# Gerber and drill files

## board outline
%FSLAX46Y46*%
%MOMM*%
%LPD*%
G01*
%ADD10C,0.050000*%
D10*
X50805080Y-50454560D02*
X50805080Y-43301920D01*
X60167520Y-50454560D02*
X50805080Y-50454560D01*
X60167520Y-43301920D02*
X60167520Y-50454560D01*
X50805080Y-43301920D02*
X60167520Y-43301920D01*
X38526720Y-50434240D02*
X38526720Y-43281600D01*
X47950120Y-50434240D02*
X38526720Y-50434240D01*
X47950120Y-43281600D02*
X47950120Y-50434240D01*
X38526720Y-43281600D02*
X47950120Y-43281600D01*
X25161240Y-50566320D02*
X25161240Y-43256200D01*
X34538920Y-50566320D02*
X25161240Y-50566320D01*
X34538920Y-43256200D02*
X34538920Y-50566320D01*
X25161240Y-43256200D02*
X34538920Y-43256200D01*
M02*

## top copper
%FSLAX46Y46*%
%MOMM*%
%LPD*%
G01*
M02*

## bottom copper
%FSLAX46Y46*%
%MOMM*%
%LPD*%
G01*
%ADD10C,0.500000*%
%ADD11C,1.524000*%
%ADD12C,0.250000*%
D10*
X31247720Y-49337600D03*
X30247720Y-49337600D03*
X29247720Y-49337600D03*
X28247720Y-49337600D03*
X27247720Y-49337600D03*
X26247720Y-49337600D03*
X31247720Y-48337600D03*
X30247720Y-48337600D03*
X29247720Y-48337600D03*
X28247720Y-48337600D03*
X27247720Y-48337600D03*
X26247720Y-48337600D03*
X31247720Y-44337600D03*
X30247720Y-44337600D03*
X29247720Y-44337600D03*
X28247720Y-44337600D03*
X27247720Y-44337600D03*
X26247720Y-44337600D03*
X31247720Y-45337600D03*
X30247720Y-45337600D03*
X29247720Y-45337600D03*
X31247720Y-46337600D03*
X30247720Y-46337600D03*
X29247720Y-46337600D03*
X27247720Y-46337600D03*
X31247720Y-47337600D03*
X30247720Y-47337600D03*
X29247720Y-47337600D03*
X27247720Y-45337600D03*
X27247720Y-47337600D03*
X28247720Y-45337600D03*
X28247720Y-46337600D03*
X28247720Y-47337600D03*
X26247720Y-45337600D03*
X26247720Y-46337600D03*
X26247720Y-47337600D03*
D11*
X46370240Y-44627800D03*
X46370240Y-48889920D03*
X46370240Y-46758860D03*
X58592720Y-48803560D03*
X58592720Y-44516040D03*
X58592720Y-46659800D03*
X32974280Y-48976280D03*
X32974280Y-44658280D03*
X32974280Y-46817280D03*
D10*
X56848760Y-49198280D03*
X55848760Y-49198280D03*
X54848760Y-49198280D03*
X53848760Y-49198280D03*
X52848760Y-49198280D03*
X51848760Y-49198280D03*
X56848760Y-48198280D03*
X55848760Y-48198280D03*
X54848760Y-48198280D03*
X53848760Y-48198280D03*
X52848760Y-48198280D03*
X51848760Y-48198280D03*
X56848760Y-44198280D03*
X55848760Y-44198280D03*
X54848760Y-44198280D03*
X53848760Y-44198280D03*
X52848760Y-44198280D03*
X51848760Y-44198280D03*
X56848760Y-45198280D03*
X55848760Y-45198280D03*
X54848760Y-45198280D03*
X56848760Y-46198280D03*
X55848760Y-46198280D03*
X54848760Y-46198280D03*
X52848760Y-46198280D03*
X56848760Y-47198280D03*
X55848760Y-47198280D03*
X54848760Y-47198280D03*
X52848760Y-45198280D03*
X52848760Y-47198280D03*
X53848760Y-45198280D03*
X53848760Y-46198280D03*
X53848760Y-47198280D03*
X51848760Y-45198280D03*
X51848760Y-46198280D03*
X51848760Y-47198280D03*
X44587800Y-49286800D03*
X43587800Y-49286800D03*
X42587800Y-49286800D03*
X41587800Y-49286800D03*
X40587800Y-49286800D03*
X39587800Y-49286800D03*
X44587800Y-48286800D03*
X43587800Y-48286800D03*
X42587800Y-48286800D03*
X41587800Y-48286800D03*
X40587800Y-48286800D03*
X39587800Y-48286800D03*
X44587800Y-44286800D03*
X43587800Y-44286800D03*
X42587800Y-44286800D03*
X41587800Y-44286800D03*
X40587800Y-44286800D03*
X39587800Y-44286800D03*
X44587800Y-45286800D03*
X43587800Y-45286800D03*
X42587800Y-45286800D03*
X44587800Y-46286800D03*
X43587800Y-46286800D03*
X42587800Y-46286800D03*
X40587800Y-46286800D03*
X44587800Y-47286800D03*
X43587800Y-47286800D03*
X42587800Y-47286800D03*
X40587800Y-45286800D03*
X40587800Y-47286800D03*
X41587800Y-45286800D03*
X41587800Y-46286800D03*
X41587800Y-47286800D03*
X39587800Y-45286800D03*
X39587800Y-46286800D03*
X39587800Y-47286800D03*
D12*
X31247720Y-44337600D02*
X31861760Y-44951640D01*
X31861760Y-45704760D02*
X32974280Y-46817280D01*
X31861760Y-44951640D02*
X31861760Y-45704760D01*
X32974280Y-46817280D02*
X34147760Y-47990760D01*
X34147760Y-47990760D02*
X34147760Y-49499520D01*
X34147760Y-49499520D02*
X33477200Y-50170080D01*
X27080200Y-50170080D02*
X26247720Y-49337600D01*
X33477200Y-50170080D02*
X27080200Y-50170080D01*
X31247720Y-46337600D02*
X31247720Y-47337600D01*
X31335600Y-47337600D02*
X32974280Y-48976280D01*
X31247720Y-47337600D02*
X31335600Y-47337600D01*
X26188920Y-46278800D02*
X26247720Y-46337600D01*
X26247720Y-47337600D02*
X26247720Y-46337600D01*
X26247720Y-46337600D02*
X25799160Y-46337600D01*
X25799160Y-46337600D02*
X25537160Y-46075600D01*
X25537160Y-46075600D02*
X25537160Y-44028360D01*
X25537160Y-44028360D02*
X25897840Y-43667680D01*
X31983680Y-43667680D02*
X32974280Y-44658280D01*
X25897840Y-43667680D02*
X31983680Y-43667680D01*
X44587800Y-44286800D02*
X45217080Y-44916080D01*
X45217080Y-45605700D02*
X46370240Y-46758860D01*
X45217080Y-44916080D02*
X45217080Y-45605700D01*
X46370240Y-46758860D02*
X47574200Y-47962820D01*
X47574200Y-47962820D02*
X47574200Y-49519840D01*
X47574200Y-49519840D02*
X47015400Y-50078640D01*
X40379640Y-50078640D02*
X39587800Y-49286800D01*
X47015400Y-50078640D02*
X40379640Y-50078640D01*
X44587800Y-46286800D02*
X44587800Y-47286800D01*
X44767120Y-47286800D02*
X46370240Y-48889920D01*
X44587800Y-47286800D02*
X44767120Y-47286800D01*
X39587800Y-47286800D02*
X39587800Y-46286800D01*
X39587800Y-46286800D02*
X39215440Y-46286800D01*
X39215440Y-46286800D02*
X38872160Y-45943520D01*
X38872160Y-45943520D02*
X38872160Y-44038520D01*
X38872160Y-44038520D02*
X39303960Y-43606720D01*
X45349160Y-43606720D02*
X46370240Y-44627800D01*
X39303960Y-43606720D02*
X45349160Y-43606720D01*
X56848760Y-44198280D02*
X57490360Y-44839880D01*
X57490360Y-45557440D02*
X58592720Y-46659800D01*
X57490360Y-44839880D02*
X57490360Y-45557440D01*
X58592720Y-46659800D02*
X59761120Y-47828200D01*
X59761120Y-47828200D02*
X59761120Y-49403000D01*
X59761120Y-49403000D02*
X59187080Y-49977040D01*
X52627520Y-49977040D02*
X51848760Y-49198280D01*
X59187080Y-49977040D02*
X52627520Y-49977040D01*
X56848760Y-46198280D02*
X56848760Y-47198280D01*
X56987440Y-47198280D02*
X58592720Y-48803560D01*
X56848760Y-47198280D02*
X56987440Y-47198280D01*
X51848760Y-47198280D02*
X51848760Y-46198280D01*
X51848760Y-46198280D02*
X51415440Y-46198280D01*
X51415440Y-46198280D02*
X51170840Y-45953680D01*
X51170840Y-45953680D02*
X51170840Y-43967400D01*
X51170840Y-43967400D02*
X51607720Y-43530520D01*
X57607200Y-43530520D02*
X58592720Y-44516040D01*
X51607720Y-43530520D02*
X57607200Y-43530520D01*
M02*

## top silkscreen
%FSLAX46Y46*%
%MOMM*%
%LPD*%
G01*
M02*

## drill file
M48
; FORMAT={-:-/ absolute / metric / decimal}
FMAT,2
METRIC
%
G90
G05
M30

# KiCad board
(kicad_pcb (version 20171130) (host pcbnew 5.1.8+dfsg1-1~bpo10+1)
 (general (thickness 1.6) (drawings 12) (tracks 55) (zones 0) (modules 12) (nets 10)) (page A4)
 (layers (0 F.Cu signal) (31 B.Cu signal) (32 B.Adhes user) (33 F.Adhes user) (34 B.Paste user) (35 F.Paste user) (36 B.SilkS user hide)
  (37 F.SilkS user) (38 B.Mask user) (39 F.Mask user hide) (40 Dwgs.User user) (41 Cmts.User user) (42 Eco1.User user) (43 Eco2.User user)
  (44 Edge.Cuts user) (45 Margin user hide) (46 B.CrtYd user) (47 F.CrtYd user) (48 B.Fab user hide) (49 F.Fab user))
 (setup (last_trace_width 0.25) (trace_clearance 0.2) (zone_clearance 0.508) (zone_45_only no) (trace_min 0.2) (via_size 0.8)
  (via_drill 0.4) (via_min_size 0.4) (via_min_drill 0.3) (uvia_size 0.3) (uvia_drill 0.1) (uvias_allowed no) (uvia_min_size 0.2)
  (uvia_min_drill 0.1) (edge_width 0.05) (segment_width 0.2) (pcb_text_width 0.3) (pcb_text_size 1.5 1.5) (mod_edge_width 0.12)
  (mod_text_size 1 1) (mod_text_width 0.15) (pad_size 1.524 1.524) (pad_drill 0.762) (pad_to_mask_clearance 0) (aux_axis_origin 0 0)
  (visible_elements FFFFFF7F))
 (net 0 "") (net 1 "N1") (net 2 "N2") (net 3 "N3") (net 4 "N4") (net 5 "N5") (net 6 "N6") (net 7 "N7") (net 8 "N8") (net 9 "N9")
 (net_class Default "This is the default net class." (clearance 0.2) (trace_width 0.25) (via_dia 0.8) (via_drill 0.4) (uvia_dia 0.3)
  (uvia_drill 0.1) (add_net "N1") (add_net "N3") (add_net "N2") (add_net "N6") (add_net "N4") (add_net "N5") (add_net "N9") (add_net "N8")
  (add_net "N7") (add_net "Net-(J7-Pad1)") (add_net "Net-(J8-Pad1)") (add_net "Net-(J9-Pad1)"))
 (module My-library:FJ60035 (layer B.Cu) (at 28.74772 46.8376)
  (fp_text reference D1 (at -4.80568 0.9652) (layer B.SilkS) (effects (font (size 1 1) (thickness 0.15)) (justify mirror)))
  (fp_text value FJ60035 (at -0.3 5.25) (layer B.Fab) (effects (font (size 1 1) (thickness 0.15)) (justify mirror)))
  (pad A6 smd circle (at 2.5 2.5) (size 0.5 0.5) (layers B.Cu B.Paste B.Mask))
  (pad A5 smd circle (at 1.5 2.5) (size 0.5 0.5) (layers B.Cu B.Paste B.Mask))
  (pad A4 smd circle (at 0.5 2.5) (size 0.5 0.5) (layers B.Cu B.Paste B.Mask))
  (pad A3 smd circle (at -0.5 2.5) (size 0.5 0.5) (layers B.Cu B.Paste B.Mask))
  (pad A2 smd circle (at -1.5 2.5) (size 0.5 0.5) (layers B.Cu B.Paste B.Mask))
  (pad A1 smd circle (at -2.5 2.5) (size 0.5 0.5) (layers B.Cu B.Paste B.Mask) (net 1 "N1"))
  (pad B6 smd circle (at 2.5 1.5) (size 0.5 0.5) (layers B.Cu B.Paste B.Mask))
  (pad B5 smd circle (at 1.5 1.5) (size 0.5 0.5) (layers B.Cu B.Paste B.Mask))
  (pad B4 smd circle (at 0.5 1.5) (size 0.5 0.5) (layers B.Cu B.Paste B.Mask))
  (pad B3 smd circle (at -0.5 1.5) (size 0.5 0.5) (layers B.Cu B.Paste B.Mask))
  (pad B2 smd circle (at -1.5 1.5) (size 0.5 0.5) (layers B.Cu B.Paste B.Mask))
  (pad B1 smd circle (at -2.5 1.5) (size 0.5 0.5) (layers B.Cu B.Paste B.Mask))
  (pad F6 smd circle (at 2.5 -2.5) (size 0.5 0.5) (layers B.Cu B.Paste B.Mask) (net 1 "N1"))
  (pad F5 smd circle (at 1.5 -2.5) (size 0.5 0.5) (layers B.Cu B.Paste B.Mask))
  (pad F4 smd circle (at 0.5 -2.5) (size 0.5 0.5) (layers B.Cu B.Paste B.Mask))
  (pad F3 smd circle (at -0.5 -2.5) (size 0.5 0.5) (layers B.Cu B.Paste B.Mask))
  (pad F2 smd circle (at -1.5 -2.5) (size 0.5 0.5) (layers B.Cu B.Paste B.Mask))
  (pad F1 smd circle (at -2.5 -2.5) (size 0.5 0.5) (layers B.Cu B.Paste B.Mask))
  (pad E6 smd circle (at 2.5 -1.5) (size 0.5 0.5) (layers B.Cu B.Paste B.Mask))
  (pad E5 smd circle (at 1.5 -1.5) (size 0.5 0.5) (layers B.Cu B.Paste B.Mask))
  (pad E4 smd circle (at 0.5 -1.5) (size 0.5 0.5) (layers B.Cu B.Paste B.Mask))
  (pad D6 smd circle (at 2.5 -0.5) (size 0.5 0.5) (layers B.Cu B.Paste B.Mask) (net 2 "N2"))
  (pad D5 smd circle (at 1.5 -0.5) (size 0.5 0.5) (layers B.Cu B.Paste B.Mask))
  (pad D4 smd circle (at 0.5 -0.5) (size 0.5 0.5) (layers B.Cu B.Paste B.Mask))
  (pad D2 smd circle (at -1.5 -0.5) (size 0.5 0.5) (layers B.Cu B.Paste B.Mask))
  (pad C6 smd circle (at 2.5 0.5) (size 0.5 0.5) (layers B.Cu B.Paste B.Mask) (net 2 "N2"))
  (pad C5 smd circle (at 1.5 0.5) (size 0.5 0.5) (layers B.Cu B.Paste B.Mask))
  (pad C4 smd circle (at 0.5 0.5) (size 0.5 0.5) (layers B.Cu B.Paste B.Mask))
  (pad E2 smd circle (at -1.5 -1.5) (size 0.5 0.5) (layers B.Cu B.Paste B.Mask))
  (pad C2 smd circle (at -1.5 0.5) (size 0.5 0.5) (layers B.Cu B.Paste B.Mask))
  (pad E3 smd circle (at -0.5 -1.5) (size 0.5 0.5) (layers B.Cu B.Paste B.Mask))
  (pad D3 smd circle (at -0.5 -0.5) (size 0.5 0.5) (layers B.Cu B.Paste B.Mask))
  (pad C3 smd circle (at -0.5 0.5) (size 0.5 0.5) (layers B.Cu B.Paste B.Mask))
  (pad E1 smd circle (at -2.5 -1.5) (size 0.5 0.5) (layers B.Cu B.Paste B.Mask))
  (pad D1 smd circle (at -2.5 -0.5) (size 0.5 0.5) (layers B.Cu B.Paste B.Mask) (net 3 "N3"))
  (pad C1 smd circle (at -2.5 0.5) (size 0.5 0.5) (layers B.Cu B.Paste B.Mask) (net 3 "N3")))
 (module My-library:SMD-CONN (layer B.Cu) (at 46.37024 44.6278)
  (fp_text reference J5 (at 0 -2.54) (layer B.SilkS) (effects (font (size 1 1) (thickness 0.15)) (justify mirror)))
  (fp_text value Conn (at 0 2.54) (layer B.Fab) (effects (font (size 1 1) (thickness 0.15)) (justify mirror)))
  (pad 1 smd circle (at 0 0) (size 1.524 1.524) (layers B.Cu B.Paste B.Mask) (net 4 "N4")))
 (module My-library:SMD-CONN (layer B.Cu) (at 46.37024 48.88992)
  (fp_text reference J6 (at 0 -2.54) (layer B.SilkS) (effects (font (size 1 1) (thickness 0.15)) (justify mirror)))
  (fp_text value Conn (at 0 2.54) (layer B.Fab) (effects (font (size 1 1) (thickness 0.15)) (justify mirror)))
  (pad 1 smd circle (at 0 0) (size 1.524 1.524) (layers B.Cu B.Paste B.Mask) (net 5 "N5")))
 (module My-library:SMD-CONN (layer B.Cu) (at 46.37024 46.5836)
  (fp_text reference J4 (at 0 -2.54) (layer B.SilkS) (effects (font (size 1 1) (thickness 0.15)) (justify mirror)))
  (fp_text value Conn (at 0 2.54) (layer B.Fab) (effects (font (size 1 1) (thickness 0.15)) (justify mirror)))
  (pad 1 smd circle (at 0 0.17526) (size 1.524 1.524) (layers B.Cu B.Paste B.Mask) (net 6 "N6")))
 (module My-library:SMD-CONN (layer B.Cu) (at 58.59272 48.80356)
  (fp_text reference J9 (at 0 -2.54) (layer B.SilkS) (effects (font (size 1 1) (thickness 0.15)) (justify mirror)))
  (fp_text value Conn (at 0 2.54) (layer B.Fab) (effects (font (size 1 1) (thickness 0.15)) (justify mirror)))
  (pad 1 smd circle (at 0 0) (size 1.524 1.524) (layers B.Cu B.Paste B.Mask) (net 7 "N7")))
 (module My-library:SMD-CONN (layer B.Cu) (at 58.59272 44.51604)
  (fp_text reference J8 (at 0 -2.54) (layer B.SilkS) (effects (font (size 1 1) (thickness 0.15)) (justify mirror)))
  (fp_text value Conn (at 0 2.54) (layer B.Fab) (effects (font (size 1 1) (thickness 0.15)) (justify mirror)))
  (pad 1 smd circle (at 0 0) (size 1.524 1.524) (layers B.Cu B.Paste B.Mask) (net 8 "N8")))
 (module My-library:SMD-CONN (layer B.Cu) (at 58.59272 46.64456)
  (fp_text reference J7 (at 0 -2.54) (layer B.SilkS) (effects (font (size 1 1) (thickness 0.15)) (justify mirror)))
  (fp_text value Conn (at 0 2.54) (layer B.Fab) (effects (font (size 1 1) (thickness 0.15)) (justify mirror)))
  (pad 1 smd circle (at 0 0.01524) (size 1.524 1.524) (layers B.Cu B.Paste B.Mask) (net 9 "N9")))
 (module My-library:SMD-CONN (layer B.Cu) (at 32.97428 48.97628)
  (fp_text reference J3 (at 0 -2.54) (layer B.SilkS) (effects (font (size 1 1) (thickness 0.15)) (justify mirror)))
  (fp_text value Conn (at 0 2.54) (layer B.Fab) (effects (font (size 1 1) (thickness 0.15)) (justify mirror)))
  (pad 1 smd circle (at 0 0) (size 1.524 1.524) (layers B.Cu B.Paste B.Mask) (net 2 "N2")))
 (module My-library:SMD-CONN (layer B.Cu) (at 32.97428 44.65828)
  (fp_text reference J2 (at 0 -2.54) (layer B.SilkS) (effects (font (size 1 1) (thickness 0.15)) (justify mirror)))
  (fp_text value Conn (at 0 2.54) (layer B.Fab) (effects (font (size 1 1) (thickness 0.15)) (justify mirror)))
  (pad 1 smd circle (at 0 0) (size 1.524 1.524) (layers B.Cu B.Paste B.Mask) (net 3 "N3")))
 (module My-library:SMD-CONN (layer B.Cu) (at 32.97428 46.94936)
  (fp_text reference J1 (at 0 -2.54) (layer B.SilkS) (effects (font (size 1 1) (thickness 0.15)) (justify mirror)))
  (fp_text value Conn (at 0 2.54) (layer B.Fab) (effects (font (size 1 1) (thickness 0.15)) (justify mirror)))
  (pad 1 smd circle (at 0 -0.13208) (size 1.524 1.524) (layers B.Cu B.Paste B.Mask) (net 1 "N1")))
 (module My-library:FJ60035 (layer B.Cu) (at 54.34876 46.69828)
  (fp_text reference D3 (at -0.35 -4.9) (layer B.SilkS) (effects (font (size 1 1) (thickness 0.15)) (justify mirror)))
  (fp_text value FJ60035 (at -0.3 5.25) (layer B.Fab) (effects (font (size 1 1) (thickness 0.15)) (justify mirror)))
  (pad A6 smd circle (at 2.5 2.5) (size 0.5 0.5) (layers B.Cu B.Paste B.Mask))
  (pad A5 smd circle (at 1.5 2.5) (size 0.5 0.5) (layers B.Cu B.Paste B.Mask))
  (pad A4 smd circle (at 0.5 2.5) (size 0.5 0.5) (layers B.Cu B.Paste B.Mask))
  (pad A3 smd circle (at -0.5 2.5) (size 0.5 0.5) (layers B.Cu B.Paste B.Mask))
  (pad A2 smd circle (at -1.5 2.5) (size 0.5 0.5) (layers B.Cu B.Paste B.Mask))
  (pad A1 smd circle (at -2.5 2.5) (size 0.5 0.5) (layers B.Cu B.Paste B.Mask) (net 9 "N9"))
  (pad B6 smd circle (at 2.5 1.5) (size 0.5 0.5) (layers B.Cu B.Paste B.Mask))
  (pad B5 smd circle (at 1.5 1.5) (size 0.5 0.5) (layers B.Cu B.Paste B.Mask))
  (pad B4 smd circle (at 0.5 1.5) (size 0.5 0.5) (layers B.Cu B.Paste B.Mask))
  (pad B3 smd circle (at -0.5 1.5) (size 0.5 0.5) (layers B.Cu B.Paste B.Mask))
  (pad B2 smd circle (at -1.5 1.5) (size 0.5 0.5) (layers B.Cu B.Paste B.Mask))
  (pad B1 smd circle (at -2.5 1.5) (size 0.5 0.5) (layers B.Cu B.Paste B.Mask))
  (pad F6 smd circle (at 2.5 -2.5) (size 0.5 0.5) (layers B.Cu B.Paste B.Mask) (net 9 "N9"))
  (pad F5 smd circle (at 1.5 -2.5) (size 0.5 0.5) (layers B.Cu B.Paste B.Mask))
  (pad F4 smd circle (at 0.5 -2.5) (size 0.5 0.5) (layers B.Cu B.Paste B.Mask))
  (pad F3 smd circle (at -0.5 -2.5) (size 0.5 0.5) (layers B.Cu B.Paste B.Mask))
  (pad F2 smd circle (at -1.5 -2.5) (size 0.5 0.5) (layers B.Cu B.Paste B.Mask))
  (pad F1 smd circle (at -2.5 -2.5) (size 0.5 0.5) (layers B.Cu B.Paste B.Mask))
  (pad E6 smd circle (at 2.5 -1.5) (size 0.5 0.5) (layers B.Cu B.Paste B.Mask))
  (pad E5 smd circle (at 1.5 -1.5) (size 0.5 0.5) (layers B.Cu B.Paste B.Mask))
  (pad E4 smd circle (at 0.5 -1.5) (size 0.5 0.5) (layers B.Cu B.Paste B.Mask))
  (pad D6 smd circle (at 2.5 -0.5) (size 0.5 0.5) (layers B.Cu B.Paste B.Mask) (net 7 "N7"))
  (pad D5 smd circle (at 1.5 -0.5) (size 0.5 0.5) (layers B.Cu B.Paste B.Mask))
  (pad D4 smd circle (at 0.5 -0.5) (size 0.5 0.5) (layers B.Cu B.Paste B.Mask))
  (pad D2 smd circle (at -1.5 -0.5) (size 0.5 0.5) (layers B.Cu B.Paste B.Mask))
  (pad C6 smd circle (at 2.5 0.5) (size 0.5 0.5) (layers B.Cu B.Paste B.Mask) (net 7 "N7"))
  (pad C5 smd circle (at 1.5 0.5) (size 0.5 0.5) (layers B.Cu B.Paste B.Mask))
  (pad C4 smd circle (at 0.5 0.5) (size 0.5 0.5) (layers B.Cu B.Paste B.Mask))
  (pad E2 smd circle (at -1.5 -1.5) (size 0.5 0.5) (layers B.Cu B.Paste B.Mask))
  (pad C2 smd circle (at -1.5 0.5) (size 0.5 0.5) (layers B.Cu B.Paste B.Mask))
  (pad E3 smd circle (at -0.5 -1.5) (size 0.5 0.5) (layers B.Cu B.Paste B.Mask))
  (pad D3 smd circle (at -0.5 -0.5) (size 0.5 0.5) (layers B.Cu B.Paste B.Mask))
  (pad C3 smd circle (at -0.5 0.5) (size 0.5 0.5) (layers B.Cu B.Paste B.Mask))
  (pad E1 smd circle (at -2.5 -1.5) (size 0.5 0.5) (layers B.Cu B.Paste B.Mask))
  (pad D1 smd circle (at -2.5 -0.5) (size 0.5 0.5) (layers B.Cu B.Paste B.Mask) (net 8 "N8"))
  (pad C1 smd circle (at -2.5 0.5) (size 0.5 0.5) (layers B.Cu B.Paste B.Mask) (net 8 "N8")))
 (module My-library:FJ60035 (layer B.Cu) (at 42.0878 46.7868)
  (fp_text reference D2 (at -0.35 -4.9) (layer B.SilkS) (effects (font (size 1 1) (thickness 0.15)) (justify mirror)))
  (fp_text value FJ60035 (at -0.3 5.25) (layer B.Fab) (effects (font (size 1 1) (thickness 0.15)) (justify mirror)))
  (pad A6 smd circle (at 2.5 2.5) (size 0.5 0.5) (layers B.Cu B.Paste B.Mask))
  (pad A5 smd circle (at 1.5 2.5) (size 0.5 0.5) (layers B.Cu B.Paste B.Mask))
  (pad A4 smd circle (at 0.5 2.5) (size 0.5 0.5) (layers B.Cu B.Paste B.Mask))
  (pad A3 smd circle (at -0.5 2.5) (size 0.5 0.5) (layers B.Cu B.Paste B.Mask))
  (pad A2 smd circle (at -1.5 2.5) (size 0.5 0.5) (layers B.Cu B.Paste B.Mask))
  (pad A1 smd circle (at -2.5 2.5) (size 0.5 0.5) (layers B.Cu B.Paste B.Mask) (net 6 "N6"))
  (pad B6 smd circle (at 2.5 1.5) (size 0.5 0.5) (layers B.Cu B.Paste B.Mask))
  (pad B5 smd circle (at 1.5 1.5) (size 0.5 0.5) (layers B.Cu B.Paste B.Mask))
  (pad B4 smd circle (at 0.5 1.5) (size 0.5 0.5) (layers B.Cu B.Paste B.Mask))
  (pad B3 smd circle (at -0.5 1.5) (size 0.5 0.5) (layers B.Cu B.Paste B.Mask))
  (pad B2 smd circle (at -1.5 1.5) (size 0.5 0.5) (layers B.Cu B.Paste B.Mask))
  (pad B1 smd circle (at -2.5 1.5) (size 0.5 0.5) (layers B.Cu B.Paste B.Mask))
  (pad F6 smd circle (at 2.5 -2.5) (size 0.5 0.5) (layers B.Cu B.Paste B.Mask) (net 6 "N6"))
  (pad F5 smd circle (at 1.5 -2.5) (size 0.5 0.5) (layers B.Cu B.Paste B.Mask))
  (pad F4 smd circle (at 0.5 -2.5) (size 0.5 0.5) (layers B.Cu B.Paste B.Mask))
  (pad F3 smd circle (at -0.5 -2.5) (size 0.5 0.5) (layers B.Cu B.Paste B.Mask))
  (pad F2 smd circle (at -1.5 -2.5) (size 0.5 0.5) (layers B.Cu B.Paste B.Mask))
  (pad F1 smd circle (at -2.5 -2.5) (size 0.5 0.5) (layers B.Cu B.Paste B.Mask))
  (pad E6 smd circle (at 2.5 -1.5) (size 0.5 0.5) (layers B.Cu B.Paste B.Mask))
  (pad E5 smd circle (at 1.5 -1.5) (size 0.5 0.5) (layers B.Cu B.Paste B.Mask))
  (pad E4 smd circle (at 0.5 -1.5) (size 0.5 0.5) (layers B.Cu B.Paste B.Mask))
  (pad D6 smd circle (at 2.5 -0.5) (size 0.5 0.5) (layers B.Cu B.Paste B.Mask) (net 5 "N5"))
  (pad D5 smd circle (at 1.5 -0.5) (size 0.5 0.5) (layers B.Cu B.Paste B.Mask))
  (pad D4 smd circle (at 0.5 -0.5) (size 0.5 0.5) (layers B.Cu B.Paste B.Mask))
  (pad D2 smd circle (at -1.5 -0.5) (size 0.5 0.5) (layers B.Cu B.Paste B.Mask))
  (pad C6 smd circle (at 2.5 0.5) (size 0.5 0.5) (layers B.Cu B.Paste B.Mask) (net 5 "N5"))
  (pad C5 smd circle (at 1.5 0.5) (size 0.5 0.5) (layers B.Cu B.Paste B.Mask))
  (pad C4 smd circle (at 0.5 0.5) (size 0.5 0.5) (layers B.Cu B.Paste B.Mask))
  (pad E2 smd circle (at -1.5 -1.5) (size 0.5 0.5) (layers B.Cu B.Paste B.Mask))
  (pad C2 smd circle (at -1.5 0.5) (size 0.5 0.5) (layers B.Cu B.Paste B.Mask))
  (pad E3 smd circle (at -0.5 -1.5) (size 0.5 0.5) (layers B.Cu B.Paste B.Mask))
  (pad D3 smd circle (at -0.5 -0.5) (size 0.5 0.5) (layers B.Cu B.Paste B.Mask))
  (pad C3 smd circle (at -0.5 0.5) (size 0.5 0.5) (layers B.Cu B.Paste B.Mask))
  (pad E1 smd circle (at -2.5 -1.5) (size 0.5 0.5) (layers B.Cu B.Paste B.Mask))
  (pad D1 smd circle (at -2.5 -0.5) (size 0.5 0.5) (layers B.Cu B.Paste B.Mask) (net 4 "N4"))
  (pad C1 smd circle (at -2.5 0.5) (size 0.5 0.5) (layers B.Cu B.Paste B.Mask) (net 4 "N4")))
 (gr_line (start 50.80508 50.45456) (end 50.80508 43.30192) (layer Edge.Cuts) (width 0.05))
 (gr_line (start 60.16752 50.45456) (end 50.80508 50.45456) (layer Edge.Cuts) (width 0.05))
 (gr_line (start 60.16752 43.30192) (end 60.16752 50.45456) (layer Edge.Cuts) (width 0.05))
 (gr_line (start 50.80508 43.30192) (end 60.16752 43.30192) (layer Edge.Cuts) (width 0.05))
 (gr_line (start 38.52672 50.43424) (end 38.52672 43.2816) (layer Edge.Cuts) (width 0.05))
 (gr_line (start 47.95012 50.43424) (end 38.52672 50.43424) (layer Edge.Cuts) (width 0.05))
 (gr_line (start 47.95012 43.2816) (end 47.95012 50.43424) (layer Edge.Cuts) (width 0.05))
 (gr_line (start 38.52672 43.2816) (end 47.95012 43.2816) (layer Edge.Cuts) (width 0.05))
 (gr_line (start 25.16124 50.56632) (end 25.16124 43.2562) (layer Edge.Cuts) (width 0.05))
 (gr_line (start 34.53892 50.56632) (end 25.16124 50.56632) (layer Edge.Cuts) (width 0.05))
 (gr_line (start 34.53892 43.2562) (end 34.53892 50.56632) (layer Edge.Cuts) (width 0.05))
 (gr_line (start 25.16124 43.2562) (end 34.53892 43.2562) (layer Edge.Cuts) (width 0.05))
 (segment (start 31.24772 44.3376) (end 31.86176 44.95164) (width 0.25) (layer B.Cu) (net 1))
 (segment (start 31.86176 45.70476) (end 32.97428 46.81728) (width 0.25) (layer B.Cu) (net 1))
 (segment (start 31.86176 44.95164) (end 31.86176 45.70476) (width 0.25) (layer B.Cu) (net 1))
 (segment (start 32.97428 46.81728) (end 34.14776 47.99076) (width 0.25) (layer B.Cu) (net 1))
 (segment (start 34.14776 47.99076) (end 34.14776 49.49952) (width 0.25) (layer B.Cu) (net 1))
 (segment (start 34.14776 49.49952) (end 33.4772 50.17008) (width 0.25) (layer B.Cu) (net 1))
 (segment (start 27.0802 50.17008) (end 26.24772 49.3376) (width 0.25) (layer B.Cu) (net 1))
 (segment (start 33.4772 50.17008) (end 27.0802 50.17008) (width 0.25) (layer B.Cu) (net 1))
 (segment (start 31.24772 46.3376) (end 31.24772 47.3376) (width 0.25) (layer B.Cu) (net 2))
 (segment (start 31.3356 47.3376) (end 32.97428 48.97628) (width 0.25) (layer B.Cu) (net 2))
 (segment (start 31.24772 47.3376) (end 31.3356 47.3376) (width 0.25) (layer B.Cu) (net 2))
 (segment (start 26.18892 46.2788) (end 26.24772 46.3376) (width 0.25) (layer B.Cu) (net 3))
 (segment (start 26.24772 47.3376) (end 26.24772 46.3376) (width 0.25) (layer B.Cu) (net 3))
 (segment (start 26.24772 46.3376) (end 25.79916 46.3376) (width 0.25) (layer B.Cu) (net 3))
 (segment (start 25.79916 46.3376) (end 25.53716 46.0756) (width 0.25) (layer B.Cu) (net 3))
 (segment (start 25.53716 46.0756) (end 25.53716 44.02836) (width 0.25) (layer B.Cu) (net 3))
 (segment (start 25.53716 44.02836) (end 25.89784 43.66768) (width 0.25) (layer B.Cu) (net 3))
 (segment (start 31.98368 43.66768) (end 32.97428 44.65828) (width 0.25) (layer B.Cu) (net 3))
 (segment (start 25.89784 43.66768) (end 31.98368 43.66768) (width 0.25) (layer B.Cu) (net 3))
 (segment (start 44.5878 44.2868) (end 45.21708 44.91608) (width 0.25) (layer B.Cu) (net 6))
 (segment (start 45.21708 45.6057) (end 46.37024 46.75886) (width 0.25) (layer B.Cu) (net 6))
 (segment (start 45.21708 44.91608) (end 45.21708 45.6057) (width 0.25) (layer B.Cu) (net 6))
 (segment (start 46.37024 46.75886) (end 47.5742 47.96282) (width 0.25) (layer B.Cu) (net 6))
 (segment (start 47.5742 47.96282) (end 47.5742 49.51984) (width 0.25) (layer B.Cu) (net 6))
 (segment (start 47.5742 49.51984) (end 47.0154 50.07864) (width 0.25) (layer B.Cu) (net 6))
 (segment (start 40.37964 50.07864) (end 39.5878 49.2868) (width 0.25) (layer B.Cu) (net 6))
 (segment (start 47.0154 50.07864) (end 40.37964 50.07864) (width 0.25) (layer B.Cu) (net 6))
 (segment (start 44.5878 46.2868) (end 44.5878 47.2868) (width 0.25) (layer B.Cu) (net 5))
 (segment (start 44.76712 47.2868) (end 46.37024 48.88992) (width 0.25) (layer B.Cu) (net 5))
 (segment (start 44.5878 47.2868) (end 44.76712 47.2868) (width 0.25) (layer B.Cu) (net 5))
 (segment (start 39.5878 47.2868) (end 39.5878 46.2868) (width 0.25) (layer B.Cu) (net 4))
 (segment (start 39.5878 46.2868) (end 39.21544 46.2868) (width 0.25) (layer B.Cu) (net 4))
 (segment (start 39.21544 46.2868) (end 38.87216 45.94352) (width 0.25) (layer B.Cu) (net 4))
 (segment (start 38.87216 45.94352) (end 38.87216 44.03852) (width 0.25) (layer B.Cu) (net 4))
 (segment (start 38.87216 44.03852) (end 39.30396 43.60672) (width 0.25) (layer B.Cu) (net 4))
 (segment (start 45.34916 43.60672) (end 46.37024 44.6278) (width 0.25) (layer B.Cu) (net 4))
 (segment (start 39.30396 43.60672) (end 45.34916 43.60672) (width 0.25) (layer B.Cu) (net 4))
 (segment (start 56.84876 44.19828) (end 57.49036 44.83988) (width 0.25) (layer B.Cu) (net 9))
 (segment (start 57.49036 45.55744) (end 58.59272 46.6598) (width 0.25) (layer B.Cu) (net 9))
 (segment (start 57.49036 44.83988) (end 57.49036 45.55744) (width 0.25) (layer B.Cu) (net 9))
 (segment (start 58.59272 46.6598) (end 59.76112 47.8282) (width 0.25) (layer B.Cu) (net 9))
 (segment (start 59.76112 47.8282) (end 59.76112 49.403) (width 0.25) (layer B.Cu) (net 9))
 (segment (start 59.76112 49.403) (end 59.18708 49.97704) (width 0.25) (layer B.Cu) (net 9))
 (segment (start 52.62752 49.97704) (end 51.84876 49.19828) (width 0.25) (layer B.Cu) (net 9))
 (segment (start 59.18708 49.97704) (end 52.62752 49.97704) (width 0.25) (layer B.Cu) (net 9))
 (segment (start 56.84876 46.19828) (end 56.84876 47.19828) (width 0.25) (layer B.Cu) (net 7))
 (segment (start 56.98744 47.19828) (end 58.59272 48.80356) (width 0.25) (layer B.Cu) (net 7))
 (segment (start 56.84876 47.19828) (end 56.98744 47.19828) (width 0.25) (layer B.Cu) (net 7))
 (segment (start 51.84876 47.19828) (end 51.84876 46.19828) (width 0.25) (layer B.Cu) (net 8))
 (segment (start 51.84876 46.19828) (end 51.41544 46.19828) (width 0.25) (layer B.Cu) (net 8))
 (segment (start 51.41544 46.19828) (end 51.17084 45.95368) (width 0.25) (layer B.Cu) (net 8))
 (segment (start 51.17084 45.95368) (end 51.17084 43.9674) (width 0.25) (layer B.Cu) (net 8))
 (segment (start 51.17084 43.9674) (end 51.60772 43.53052) (width 0.25) (layer B.Cu) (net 8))
 (segment (start 57.6072 43.53052) (end 58.59272 44.51604) (width 0.25) (layer B.Cu) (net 8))
 (segment (start 51.60772 43.53052) (end 57.6072 43.53052) (width 0.25) (layer B.Cu) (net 8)))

